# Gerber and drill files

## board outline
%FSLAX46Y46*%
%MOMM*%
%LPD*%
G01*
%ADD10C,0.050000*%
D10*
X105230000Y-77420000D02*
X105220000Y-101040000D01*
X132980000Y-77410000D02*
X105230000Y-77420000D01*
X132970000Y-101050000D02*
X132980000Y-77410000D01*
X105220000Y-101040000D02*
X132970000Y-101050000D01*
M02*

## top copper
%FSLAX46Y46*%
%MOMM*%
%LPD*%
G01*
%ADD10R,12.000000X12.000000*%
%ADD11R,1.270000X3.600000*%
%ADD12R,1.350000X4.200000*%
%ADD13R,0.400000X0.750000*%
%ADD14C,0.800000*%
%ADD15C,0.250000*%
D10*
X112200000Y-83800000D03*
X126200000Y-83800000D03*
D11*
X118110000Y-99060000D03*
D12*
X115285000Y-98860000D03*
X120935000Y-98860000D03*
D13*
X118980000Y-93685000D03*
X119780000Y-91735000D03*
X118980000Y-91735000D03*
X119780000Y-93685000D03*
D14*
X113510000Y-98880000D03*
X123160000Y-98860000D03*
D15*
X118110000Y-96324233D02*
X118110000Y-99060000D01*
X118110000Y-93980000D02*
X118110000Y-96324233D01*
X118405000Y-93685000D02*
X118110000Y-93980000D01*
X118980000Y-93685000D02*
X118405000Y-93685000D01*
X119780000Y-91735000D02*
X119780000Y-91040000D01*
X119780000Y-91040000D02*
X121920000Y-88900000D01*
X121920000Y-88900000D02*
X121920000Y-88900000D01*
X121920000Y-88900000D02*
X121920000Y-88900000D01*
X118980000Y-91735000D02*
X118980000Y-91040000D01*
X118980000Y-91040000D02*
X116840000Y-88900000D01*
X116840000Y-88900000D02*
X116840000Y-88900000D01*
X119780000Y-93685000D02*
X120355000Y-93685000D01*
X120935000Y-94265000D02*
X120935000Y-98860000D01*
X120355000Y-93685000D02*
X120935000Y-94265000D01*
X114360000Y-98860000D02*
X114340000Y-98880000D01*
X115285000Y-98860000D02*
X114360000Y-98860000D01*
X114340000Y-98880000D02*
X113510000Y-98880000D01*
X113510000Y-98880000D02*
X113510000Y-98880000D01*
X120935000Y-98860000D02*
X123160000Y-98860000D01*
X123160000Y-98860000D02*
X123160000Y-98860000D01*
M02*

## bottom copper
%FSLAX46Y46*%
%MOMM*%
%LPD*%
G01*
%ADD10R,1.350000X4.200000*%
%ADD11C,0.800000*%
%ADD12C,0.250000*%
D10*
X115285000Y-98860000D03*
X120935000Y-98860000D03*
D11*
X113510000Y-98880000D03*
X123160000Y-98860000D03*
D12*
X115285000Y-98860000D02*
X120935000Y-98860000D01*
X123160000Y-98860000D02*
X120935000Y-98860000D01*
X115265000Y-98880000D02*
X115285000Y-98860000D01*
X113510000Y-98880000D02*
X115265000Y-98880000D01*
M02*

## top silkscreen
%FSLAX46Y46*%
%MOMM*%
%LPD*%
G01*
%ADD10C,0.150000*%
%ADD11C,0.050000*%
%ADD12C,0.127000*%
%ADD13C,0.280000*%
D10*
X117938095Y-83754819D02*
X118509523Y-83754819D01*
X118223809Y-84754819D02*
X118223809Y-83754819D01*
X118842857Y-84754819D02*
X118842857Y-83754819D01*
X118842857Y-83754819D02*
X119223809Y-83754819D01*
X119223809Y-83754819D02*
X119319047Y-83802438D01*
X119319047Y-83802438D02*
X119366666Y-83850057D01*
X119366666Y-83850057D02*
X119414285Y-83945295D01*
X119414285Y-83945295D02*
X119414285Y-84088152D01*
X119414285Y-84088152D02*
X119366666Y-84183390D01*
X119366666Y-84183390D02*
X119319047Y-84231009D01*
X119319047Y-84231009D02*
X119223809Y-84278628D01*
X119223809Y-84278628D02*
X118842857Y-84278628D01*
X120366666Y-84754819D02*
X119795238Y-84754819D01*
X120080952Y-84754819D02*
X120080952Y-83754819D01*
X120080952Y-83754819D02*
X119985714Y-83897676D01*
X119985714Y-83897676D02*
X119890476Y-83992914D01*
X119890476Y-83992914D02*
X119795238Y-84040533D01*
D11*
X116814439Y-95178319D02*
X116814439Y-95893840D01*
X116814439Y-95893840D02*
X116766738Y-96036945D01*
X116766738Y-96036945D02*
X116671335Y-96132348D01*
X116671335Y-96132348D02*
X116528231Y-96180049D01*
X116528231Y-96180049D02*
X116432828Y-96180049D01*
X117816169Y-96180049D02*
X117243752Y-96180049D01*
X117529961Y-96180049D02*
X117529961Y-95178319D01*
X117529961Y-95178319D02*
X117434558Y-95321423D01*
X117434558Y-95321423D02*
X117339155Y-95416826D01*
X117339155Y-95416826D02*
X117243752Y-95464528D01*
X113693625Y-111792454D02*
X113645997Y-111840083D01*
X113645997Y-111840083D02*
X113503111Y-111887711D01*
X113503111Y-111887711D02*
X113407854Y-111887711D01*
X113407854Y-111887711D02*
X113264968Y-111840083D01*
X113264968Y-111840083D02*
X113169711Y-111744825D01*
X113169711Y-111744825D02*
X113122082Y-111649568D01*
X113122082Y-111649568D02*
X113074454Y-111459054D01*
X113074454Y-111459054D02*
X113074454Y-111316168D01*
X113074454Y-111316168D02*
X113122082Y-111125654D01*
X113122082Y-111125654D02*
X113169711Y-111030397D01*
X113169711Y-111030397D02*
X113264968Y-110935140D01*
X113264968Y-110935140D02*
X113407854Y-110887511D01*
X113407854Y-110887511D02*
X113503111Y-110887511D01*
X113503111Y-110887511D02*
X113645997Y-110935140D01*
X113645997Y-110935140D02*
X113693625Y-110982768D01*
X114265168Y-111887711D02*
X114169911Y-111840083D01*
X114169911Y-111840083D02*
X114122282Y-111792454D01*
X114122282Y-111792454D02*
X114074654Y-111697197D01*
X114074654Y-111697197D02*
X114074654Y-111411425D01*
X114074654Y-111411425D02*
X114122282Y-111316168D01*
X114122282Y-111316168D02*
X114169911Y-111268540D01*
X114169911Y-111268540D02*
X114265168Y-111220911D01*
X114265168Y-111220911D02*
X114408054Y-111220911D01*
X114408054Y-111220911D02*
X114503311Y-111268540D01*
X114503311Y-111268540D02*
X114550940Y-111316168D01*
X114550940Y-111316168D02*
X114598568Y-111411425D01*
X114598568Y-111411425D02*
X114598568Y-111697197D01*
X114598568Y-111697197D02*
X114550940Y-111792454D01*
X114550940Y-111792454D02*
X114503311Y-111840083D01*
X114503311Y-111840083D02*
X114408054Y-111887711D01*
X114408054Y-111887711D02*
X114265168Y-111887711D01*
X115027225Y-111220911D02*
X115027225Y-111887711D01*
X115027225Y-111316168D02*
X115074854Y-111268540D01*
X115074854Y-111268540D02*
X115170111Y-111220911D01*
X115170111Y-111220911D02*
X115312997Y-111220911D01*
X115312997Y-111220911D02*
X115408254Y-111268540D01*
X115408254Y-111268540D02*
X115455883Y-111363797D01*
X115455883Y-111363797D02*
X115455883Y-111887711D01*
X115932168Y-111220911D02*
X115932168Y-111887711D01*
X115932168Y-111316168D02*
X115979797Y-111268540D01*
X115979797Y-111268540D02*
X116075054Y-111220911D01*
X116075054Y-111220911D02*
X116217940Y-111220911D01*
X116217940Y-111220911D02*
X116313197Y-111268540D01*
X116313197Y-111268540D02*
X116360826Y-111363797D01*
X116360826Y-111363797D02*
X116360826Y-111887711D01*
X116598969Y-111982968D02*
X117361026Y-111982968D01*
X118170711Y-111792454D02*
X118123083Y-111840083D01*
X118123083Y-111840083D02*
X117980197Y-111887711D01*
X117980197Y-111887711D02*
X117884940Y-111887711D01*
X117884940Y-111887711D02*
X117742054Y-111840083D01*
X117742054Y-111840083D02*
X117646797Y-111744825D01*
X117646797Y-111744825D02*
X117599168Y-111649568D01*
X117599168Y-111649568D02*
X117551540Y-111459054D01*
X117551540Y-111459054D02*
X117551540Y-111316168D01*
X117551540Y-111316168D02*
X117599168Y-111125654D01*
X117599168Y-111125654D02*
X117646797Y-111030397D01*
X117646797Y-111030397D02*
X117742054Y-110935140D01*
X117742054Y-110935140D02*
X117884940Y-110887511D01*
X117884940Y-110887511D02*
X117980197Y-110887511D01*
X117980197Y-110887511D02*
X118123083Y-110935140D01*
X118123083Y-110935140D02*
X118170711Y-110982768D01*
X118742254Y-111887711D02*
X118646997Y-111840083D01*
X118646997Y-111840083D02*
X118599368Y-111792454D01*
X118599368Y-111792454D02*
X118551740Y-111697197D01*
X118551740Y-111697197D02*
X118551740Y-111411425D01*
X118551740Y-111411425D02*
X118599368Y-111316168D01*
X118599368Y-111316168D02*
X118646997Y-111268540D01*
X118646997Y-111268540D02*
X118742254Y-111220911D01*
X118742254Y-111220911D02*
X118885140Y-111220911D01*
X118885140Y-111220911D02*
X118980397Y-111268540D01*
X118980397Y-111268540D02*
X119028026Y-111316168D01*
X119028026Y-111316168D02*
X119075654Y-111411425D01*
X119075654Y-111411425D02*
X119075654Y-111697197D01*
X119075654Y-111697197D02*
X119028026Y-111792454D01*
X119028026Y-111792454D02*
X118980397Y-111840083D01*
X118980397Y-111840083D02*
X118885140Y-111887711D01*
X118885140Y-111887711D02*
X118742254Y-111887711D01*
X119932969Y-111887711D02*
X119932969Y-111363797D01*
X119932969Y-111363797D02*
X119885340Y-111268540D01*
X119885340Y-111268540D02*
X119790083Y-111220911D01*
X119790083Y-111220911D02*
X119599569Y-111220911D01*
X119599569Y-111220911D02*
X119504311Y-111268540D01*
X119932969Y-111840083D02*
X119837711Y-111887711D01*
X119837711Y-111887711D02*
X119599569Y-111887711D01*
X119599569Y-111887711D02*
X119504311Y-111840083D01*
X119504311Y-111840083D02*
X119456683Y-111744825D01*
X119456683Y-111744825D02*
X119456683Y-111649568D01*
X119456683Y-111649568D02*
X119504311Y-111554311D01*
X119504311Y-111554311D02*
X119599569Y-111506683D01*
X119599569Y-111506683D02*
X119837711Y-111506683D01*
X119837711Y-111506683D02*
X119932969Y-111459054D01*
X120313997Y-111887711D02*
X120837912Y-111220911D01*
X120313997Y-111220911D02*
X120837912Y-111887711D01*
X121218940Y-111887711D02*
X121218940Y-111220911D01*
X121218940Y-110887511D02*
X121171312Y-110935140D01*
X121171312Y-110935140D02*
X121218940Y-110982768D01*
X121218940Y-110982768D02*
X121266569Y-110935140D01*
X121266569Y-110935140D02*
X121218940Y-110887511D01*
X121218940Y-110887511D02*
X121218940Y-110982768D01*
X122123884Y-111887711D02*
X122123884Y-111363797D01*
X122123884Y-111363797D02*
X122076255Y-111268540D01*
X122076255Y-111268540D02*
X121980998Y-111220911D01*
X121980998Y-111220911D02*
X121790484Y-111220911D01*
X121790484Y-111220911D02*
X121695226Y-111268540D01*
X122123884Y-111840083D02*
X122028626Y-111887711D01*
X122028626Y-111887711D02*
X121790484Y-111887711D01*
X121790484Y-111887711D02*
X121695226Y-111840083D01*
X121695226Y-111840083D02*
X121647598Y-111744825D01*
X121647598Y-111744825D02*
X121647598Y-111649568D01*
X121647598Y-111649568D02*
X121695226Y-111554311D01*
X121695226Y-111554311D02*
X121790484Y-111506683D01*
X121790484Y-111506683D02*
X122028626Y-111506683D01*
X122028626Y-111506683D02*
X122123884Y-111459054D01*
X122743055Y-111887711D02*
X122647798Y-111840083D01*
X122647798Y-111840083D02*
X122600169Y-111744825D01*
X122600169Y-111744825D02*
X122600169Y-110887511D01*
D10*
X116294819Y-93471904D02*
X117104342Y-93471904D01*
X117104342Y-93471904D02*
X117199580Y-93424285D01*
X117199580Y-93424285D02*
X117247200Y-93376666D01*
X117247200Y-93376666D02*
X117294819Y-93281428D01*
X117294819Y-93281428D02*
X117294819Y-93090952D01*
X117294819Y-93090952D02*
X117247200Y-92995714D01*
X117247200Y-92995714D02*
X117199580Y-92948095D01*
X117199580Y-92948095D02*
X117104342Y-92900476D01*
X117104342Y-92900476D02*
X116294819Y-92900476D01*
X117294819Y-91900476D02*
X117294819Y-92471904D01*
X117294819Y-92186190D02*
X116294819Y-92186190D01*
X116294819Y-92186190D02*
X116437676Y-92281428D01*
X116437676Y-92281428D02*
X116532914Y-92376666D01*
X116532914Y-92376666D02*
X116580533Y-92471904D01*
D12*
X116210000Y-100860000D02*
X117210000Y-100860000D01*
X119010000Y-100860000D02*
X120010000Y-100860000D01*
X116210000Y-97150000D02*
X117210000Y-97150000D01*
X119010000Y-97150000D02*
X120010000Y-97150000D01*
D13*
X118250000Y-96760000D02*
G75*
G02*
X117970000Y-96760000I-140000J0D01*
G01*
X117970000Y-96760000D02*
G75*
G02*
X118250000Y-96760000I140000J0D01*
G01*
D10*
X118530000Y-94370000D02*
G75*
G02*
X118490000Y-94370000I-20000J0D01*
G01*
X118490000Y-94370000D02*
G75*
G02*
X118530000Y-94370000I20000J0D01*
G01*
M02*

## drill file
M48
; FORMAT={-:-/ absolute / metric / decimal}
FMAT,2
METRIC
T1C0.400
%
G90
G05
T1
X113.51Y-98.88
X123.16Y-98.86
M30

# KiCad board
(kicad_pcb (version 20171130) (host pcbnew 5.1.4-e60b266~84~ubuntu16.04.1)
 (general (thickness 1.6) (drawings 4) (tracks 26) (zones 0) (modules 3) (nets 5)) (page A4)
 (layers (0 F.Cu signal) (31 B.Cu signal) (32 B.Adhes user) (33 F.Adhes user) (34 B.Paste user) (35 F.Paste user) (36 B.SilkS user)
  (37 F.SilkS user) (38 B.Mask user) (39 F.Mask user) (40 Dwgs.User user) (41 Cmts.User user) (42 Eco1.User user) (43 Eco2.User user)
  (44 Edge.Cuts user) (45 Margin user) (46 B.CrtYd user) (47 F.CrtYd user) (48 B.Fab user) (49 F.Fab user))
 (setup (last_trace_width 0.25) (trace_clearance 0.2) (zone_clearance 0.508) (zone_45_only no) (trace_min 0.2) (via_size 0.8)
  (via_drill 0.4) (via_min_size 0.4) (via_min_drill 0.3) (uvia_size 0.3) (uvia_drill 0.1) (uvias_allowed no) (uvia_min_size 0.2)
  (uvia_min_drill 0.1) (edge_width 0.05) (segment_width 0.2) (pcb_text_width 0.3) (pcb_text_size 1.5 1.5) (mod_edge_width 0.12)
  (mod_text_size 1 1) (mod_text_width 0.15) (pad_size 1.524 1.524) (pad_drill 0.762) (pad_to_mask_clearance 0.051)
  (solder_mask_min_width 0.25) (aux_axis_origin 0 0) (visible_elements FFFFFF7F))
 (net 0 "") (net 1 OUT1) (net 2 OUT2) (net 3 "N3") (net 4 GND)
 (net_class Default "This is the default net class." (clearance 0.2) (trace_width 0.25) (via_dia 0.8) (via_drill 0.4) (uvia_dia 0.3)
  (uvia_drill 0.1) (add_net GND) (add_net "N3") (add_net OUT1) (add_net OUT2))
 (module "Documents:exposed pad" (layer F.Cu) (at 119.2 83.8)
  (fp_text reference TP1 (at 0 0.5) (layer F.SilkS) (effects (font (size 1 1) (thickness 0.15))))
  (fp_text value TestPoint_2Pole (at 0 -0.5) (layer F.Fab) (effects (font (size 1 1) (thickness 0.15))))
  (pad 1 smd rect (at -7 0) (size 12 12) (layers F.Cu F.Paste F.Mask) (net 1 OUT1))
  (pad 2 smd rect (at 7 0) (size 12 12) (layers F.Cu F.Paste F.Mask) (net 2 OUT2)))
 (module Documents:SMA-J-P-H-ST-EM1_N (layer F.Cu) (at 118.11 99.06)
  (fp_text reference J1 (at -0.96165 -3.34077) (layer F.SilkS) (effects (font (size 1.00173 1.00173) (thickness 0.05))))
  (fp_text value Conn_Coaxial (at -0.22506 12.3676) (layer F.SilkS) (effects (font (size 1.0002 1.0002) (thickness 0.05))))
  (fp_line (start -1.9 1.8) (end -0.9 1.8) (layer F.SilkS) (width 0.127))
  (fp_line (start 0.9 1.8) (end 1.9 1.8) (layer F.SilkS) (width 0.127))
  (fp_line (start -1.9 -1.91) (end -0.9 -1.91) (layer F.SilkS) (width 0.127))
  (fp_line (start 0.9 -1.91) (end 1.9 -1.91) (layer F.SilkS) (width 0.127))
  (fp_circle (center 0 -2.3) (end 0.14 -2.3) (layer F.SilkS) (width 0.28))
  (pad 1 smd rect (at 0 0) (size 1.27 3.6) (layers F.Cu F.Paste F.Mask) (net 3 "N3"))
  (pad 2 smd rect (at -2.825 -0.2) (size 1.35 4.2) (layers F.Cu F.Paste F.Mask) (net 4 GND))
  (pad 2 smd rect (at 2.825 -0.2) (size 1.35 4.2) (layers F.Cu F.Paste F.Mask) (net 4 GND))
  (pad 2 smd rect (at -2.825 -0.2) (size 1.35 4.2) (layers B.Cu F.Paste F.Mask) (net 4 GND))
  (pad 2 smd rect (at 2.825 -0.2) (size 1.35 4.2) (layers B.Cu F.Paste F.Mask) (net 4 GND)))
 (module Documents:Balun (layer F.Cu) (at 119.38 92.71 90)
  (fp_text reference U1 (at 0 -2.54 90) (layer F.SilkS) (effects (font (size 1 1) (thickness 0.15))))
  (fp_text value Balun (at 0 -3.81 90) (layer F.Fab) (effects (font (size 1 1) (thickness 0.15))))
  (fp_circle (center -1.66 -0.87) (end -1.66 -0.89) (layer F.SilkS) (width 0.15))
  (pad 1 smd rect (at -0.975 -0.4 90) (size 0.75 0.4) (layers F.Cu F.Paste F.Mask) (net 3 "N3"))
  (pad 3 smd rect (at 0.975 0.4 90) (size 0.75 0.4) (layers F.Cu F.Paste F.Mask) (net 2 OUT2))
  (pad 4 smd rect (at 0.975 -0.4 90) (size 0.75 0.4) (layers F.Cu F.Paste F.Mask) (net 1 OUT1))
  (pad 2 smd rect (at -0.975 0.4 90) (size 0.75 0.4) (layers F.Cu F.Paste F.Mask) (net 4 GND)))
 (gr_line (start 105.23 77.42) (end 105.22 101.04) (layer Edge.Cuts) (width 0.05))
 (gr_line (start 132.98 77.41) (end 105.23 77.42) (layer Edge.Cuts) (width 0.05))
 (gr_line (start 132.97 101.05) (end 132.98 77.41) (layer Edge.Cuts) (width 0.05))
 (gr_line (start 105.22 101.04) (end 132.97 101.05) (layer Edge.Cuts) (width 0.05))
 (segment (start 118.11 96.324233) (end 118.11 99.06) (width 0.25) (layer F.Cu) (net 3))
 (segment (start 118.11 93.98) (end 118.11 96.324233) (width 0.25) (layer F.Cu) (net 3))
 (segment (start 118.405 93.685) (end 118.11 93.98) (width 0.25) (layer F.Cu) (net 3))
 (segment (start 118.98 93.685) (end 118.405 93.685) (width 0.25) (layer F.Cu) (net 3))
 (segment (start 119.78 91.735) (end 119.78 91.04) (width 0.25) (layer F.Cu) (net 2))
 (segment (start 119.78 91.04) (end 121.92 88.9) (width 0.25) (layer F.Cu) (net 2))
 (segment (start 121.92 88.9) (end 121.92 88.9) (width 0.25) (layer F.Cu) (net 2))
 (segment (start 121.92 88.9) (end 121.92 88.9) (width 0.25) (layer F.Cu) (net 2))
 (segment (start 118.98 91.735) (end 118.98 91.04) (width 0.25) (layer F.Cu) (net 1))
 (segment (start 118.98 91.04) (end 116.84 88.9) (width 0.25) (layer F.Cu) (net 1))
 (segment (start 116.84 88.9) (end 116.84 88.9) (width 0.25) (layer F.Cu) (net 1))
 (segment (start 119.78 93.685) (end 120.355 93.685) (width 0.25) (layer F.Cu) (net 4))
 (segment (start 120.935 94.265) (end 120.935 98.86) (width 0.25) (layer F.Cu) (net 4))
 (segment (start 120.355 93.685) (end 120.935 94.265) (width 0.25) (layer F.Cu) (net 4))
 (segment (start 115.285 98.86) (end 120.935 98.86) (width 0.25) (layer B.Cu) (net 4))
 (segment (start 114.36 98.86) (end 114.34 98.88) (width 0.25) (layer F.Cu) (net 4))
 (segment (start 115.285 98.86) (end 114.36 98.86) (width 0.25) (layer F.Cu) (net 4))
 (segment (start 114.34 98.88) (end 113.51 98.88) (width 0.25) (layer F.Cu) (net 4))
 (segment (start 113.51 98.88) (end 113.51 98.88) (width 0.25) (layer F.Cu) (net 4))
 (via (at 113.51 98.88) (size 0.8) (drill 0.4) (layers F.Cu B.Cu) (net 4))
 (segment (start 120.935 98.86) (end 123.16 98.86) (width 0.25) (layer F.Cu) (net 4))
 (segment (start 123.16 98.86) (end 123.16 98.86) (width 0.25) (layer F.Cu) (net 4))
 (via (at 123.16 98.86) (size 0.8) (drill 0.4) (layers F.Cu B.Cu) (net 4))
 (segment (start 123.16 98.86) (end 120.935 98.86) (width 0.25) (layer B.Cu) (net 4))
 (segment (start 115.265 98.88) (end 115.285 98.86) (width 0.25) (layer B.Cu) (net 4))
 (segment (start 113.51 98.88) (end 115.265 98.88) (width 0.25) (layer B.Cu) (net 4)))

